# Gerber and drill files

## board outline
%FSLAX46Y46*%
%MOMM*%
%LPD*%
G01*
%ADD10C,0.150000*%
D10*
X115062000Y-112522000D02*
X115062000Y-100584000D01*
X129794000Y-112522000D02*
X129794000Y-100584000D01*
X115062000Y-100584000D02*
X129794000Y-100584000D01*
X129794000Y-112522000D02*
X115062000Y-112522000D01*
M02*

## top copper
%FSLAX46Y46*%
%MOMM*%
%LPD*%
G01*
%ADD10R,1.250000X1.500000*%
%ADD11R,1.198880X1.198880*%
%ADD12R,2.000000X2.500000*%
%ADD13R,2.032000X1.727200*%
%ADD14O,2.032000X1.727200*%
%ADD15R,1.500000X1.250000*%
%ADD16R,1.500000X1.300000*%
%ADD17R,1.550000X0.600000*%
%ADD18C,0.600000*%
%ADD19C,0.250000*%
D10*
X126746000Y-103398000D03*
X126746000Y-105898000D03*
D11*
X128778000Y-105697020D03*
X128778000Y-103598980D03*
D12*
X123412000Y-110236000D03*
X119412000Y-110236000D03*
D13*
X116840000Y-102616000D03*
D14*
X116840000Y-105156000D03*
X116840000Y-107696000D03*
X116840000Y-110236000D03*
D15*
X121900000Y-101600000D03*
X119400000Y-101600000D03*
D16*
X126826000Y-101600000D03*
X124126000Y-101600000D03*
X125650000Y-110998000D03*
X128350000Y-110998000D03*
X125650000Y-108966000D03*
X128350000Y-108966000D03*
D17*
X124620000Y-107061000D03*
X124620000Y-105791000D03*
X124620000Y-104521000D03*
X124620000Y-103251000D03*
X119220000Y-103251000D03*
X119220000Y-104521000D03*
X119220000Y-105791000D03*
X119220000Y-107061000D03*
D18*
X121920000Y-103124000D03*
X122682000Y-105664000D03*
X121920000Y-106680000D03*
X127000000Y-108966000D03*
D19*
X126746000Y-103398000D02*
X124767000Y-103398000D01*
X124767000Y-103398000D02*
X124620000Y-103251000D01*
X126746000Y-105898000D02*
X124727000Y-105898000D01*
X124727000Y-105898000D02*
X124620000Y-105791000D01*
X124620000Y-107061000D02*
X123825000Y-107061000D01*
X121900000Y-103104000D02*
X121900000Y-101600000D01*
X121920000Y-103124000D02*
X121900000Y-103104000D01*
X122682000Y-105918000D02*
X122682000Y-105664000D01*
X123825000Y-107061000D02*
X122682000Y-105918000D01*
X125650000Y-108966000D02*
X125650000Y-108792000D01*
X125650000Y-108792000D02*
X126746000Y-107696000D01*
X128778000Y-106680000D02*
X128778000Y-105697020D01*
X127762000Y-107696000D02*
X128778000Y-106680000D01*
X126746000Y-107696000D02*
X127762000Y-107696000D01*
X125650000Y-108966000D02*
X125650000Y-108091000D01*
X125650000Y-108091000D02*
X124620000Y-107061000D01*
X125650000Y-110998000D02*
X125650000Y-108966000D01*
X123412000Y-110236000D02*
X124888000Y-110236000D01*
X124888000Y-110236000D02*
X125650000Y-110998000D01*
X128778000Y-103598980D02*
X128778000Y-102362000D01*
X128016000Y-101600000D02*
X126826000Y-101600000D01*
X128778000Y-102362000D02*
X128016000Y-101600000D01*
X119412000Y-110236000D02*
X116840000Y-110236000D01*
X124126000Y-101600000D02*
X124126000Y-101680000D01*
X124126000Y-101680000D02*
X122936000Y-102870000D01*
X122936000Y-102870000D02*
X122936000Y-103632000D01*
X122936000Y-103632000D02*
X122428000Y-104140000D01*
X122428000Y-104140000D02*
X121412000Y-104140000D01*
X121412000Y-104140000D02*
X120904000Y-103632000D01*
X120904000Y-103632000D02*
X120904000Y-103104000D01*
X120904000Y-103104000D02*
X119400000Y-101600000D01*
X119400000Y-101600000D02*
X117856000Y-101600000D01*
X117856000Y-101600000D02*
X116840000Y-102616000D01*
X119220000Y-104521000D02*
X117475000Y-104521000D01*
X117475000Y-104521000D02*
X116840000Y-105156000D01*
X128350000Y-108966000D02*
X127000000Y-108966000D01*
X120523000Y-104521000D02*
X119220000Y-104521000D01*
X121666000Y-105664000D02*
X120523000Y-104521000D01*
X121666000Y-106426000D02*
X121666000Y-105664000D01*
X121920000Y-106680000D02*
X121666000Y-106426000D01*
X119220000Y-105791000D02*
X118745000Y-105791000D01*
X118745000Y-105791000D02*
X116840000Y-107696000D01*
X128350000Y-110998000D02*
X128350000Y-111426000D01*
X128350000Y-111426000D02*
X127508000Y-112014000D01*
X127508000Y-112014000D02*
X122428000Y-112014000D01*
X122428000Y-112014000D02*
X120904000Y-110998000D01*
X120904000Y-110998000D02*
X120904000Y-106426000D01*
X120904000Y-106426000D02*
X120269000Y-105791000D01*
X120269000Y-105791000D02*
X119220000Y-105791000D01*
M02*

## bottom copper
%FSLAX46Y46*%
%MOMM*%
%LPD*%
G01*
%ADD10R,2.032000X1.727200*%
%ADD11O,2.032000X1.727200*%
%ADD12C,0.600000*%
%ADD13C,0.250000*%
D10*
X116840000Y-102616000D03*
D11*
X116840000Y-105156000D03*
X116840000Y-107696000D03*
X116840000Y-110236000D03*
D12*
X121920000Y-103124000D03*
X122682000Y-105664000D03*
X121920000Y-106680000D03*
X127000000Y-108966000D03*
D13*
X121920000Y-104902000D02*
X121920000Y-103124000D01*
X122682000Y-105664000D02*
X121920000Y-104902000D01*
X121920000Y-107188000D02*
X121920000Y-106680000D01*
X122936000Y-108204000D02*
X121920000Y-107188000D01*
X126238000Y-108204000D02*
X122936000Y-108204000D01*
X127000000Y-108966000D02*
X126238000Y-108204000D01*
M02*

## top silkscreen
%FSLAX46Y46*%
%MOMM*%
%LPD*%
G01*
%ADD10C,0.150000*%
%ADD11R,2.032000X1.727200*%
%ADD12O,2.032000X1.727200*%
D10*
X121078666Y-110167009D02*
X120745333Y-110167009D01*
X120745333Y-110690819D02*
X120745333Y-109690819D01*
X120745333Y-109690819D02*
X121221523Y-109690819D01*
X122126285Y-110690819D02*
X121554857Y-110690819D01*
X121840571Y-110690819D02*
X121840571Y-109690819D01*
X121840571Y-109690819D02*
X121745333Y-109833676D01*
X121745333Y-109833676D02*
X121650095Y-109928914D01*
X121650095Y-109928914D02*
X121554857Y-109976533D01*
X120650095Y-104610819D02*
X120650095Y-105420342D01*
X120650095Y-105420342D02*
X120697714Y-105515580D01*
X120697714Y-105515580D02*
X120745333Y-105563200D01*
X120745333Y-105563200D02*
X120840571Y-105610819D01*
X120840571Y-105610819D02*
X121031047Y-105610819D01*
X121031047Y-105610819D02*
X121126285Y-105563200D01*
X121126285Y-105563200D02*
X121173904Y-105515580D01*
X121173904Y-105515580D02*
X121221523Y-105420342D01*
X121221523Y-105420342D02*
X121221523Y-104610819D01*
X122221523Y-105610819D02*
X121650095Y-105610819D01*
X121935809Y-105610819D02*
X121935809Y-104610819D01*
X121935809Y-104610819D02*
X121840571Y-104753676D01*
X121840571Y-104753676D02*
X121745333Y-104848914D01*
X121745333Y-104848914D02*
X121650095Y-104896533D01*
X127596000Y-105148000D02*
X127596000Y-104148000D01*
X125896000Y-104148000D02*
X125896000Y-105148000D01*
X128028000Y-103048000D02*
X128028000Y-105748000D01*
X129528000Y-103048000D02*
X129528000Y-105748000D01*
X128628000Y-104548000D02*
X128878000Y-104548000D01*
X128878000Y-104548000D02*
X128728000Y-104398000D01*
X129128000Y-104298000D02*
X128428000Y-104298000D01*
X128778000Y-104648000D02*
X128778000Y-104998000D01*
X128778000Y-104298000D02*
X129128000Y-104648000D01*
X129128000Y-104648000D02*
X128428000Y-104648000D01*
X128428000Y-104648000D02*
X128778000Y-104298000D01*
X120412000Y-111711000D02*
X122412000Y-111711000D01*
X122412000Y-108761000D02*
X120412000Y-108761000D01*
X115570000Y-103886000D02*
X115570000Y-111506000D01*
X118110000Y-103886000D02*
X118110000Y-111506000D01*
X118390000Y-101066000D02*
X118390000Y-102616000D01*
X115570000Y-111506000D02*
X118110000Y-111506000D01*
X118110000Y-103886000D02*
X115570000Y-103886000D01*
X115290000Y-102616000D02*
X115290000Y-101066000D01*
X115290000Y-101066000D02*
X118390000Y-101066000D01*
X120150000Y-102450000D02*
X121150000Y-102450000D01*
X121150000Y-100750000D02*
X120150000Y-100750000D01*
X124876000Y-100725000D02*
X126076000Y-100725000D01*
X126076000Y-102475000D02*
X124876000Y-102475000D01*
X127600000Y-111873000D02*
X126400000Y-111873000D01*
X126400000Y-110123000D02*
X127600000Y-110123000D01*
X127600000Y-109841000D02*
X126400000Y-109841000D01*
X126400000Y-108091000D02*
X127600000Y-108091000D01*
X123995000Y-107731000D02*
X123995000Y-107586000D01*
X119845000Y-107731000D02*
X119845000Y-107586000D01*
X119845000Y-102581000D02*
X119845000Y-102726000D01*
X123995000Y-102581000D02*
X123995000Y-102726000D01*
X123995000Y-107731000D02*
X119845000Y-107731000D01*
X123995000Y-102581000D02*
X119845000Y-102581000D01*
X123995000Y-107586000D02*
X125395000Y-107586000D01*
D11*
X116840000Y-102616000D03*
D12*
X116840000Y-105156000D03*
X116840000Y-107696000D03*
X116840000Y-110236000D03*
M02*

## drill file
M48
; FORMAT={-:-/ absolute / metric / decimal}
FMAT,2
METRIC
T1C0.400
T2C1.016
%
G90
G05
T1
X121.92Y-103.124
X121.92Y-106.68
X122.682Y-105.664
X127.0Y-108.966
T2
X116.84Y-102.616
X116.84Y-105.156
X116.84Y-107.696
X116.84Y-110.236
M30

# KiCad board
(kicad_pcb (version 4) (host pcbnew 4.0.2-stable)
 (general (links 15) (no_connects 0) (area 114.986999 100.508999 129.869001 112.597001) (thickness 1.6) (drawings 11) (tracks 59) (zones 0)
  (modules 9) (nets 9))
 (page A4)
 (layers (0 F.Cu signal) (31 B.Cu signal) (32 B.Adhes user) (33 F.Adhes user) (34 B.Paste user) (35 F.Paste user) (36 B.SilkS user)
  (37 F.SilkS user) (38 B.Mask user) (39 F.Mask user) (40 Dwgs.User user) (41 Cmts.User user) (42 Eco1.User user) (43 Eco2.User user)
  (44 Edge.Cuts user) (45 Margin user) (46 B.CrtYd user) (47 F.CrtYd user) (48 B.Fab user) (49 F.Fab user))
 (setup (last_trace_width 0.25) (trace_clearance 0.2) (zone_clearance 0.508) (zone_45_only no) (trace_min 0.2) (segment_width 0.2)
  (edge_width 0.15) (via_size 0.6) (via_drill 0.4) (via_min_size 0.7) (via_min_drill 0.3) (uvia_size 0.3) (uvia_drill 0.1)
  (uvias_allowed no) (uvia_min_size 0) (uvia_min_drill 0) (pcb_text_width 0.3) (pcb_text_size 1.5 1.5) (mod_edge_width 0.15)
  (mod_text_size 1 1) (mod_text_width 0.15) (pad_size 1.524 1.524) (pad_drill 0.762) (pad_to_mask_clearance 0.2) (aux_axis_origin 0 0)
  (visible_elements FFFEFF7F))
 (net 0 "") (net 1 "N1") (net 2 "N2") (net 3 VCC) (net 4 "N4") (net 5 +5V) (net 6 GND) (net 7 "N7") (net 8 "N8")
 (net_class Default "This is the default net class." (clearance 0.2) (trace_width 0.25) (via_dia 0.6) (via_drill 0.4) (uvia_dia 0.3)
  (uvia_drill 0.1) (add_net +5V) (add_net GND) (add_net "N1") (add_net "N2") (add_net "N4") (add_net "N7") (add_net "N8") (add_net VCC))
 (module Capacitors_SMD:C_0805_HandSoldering (layer F.Cu) (at 126.746 104.648 270)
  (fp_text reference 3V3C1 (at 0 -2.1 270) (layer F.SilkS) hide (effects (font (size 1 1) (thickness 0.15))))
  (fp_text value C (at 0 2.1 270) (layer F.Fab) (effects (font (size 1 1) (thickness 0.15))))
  (fp_line (start 0.5 -0.85) (end -0.5 -0.85) (layer F.SilkS) (width 0.15))
  (fp_line (start -0.5 0.85) (end 0.5 0.85) (layer F.SilkS) (width 0.15))
  (pad 1 smd rect (at -1.25 0 270) (size 1.5 1.25) (layers F.Cu F.Paste F.Mask) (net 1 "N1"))
  (pad 2 smd rect (at 1.25 0 270) (size 1.5 1.25) (layers F.Cu F.Paste F.Mask) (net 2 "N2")))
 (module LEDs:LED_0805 (layer F.Cu) (at 128.778 104.648 270)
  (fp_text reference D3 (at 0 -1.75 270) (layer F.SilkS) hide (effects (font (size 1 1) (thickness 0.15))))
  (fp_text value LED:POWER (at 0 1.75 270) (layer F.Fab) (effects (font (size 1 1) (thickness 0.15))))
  (fp_line (start -1.6 0.75) (end 1.1 0.75) (layer F.SilkS) (width 0.15))
  (fp_line (start -1.6 -0.75) (end 1.1 -0.75) (layer F.SilkS) (width 0.15))
  (fp_line (start -0.1 0.15) (end -0.1 -0.1) (layer F.SilkS) (width 0.15))
  (fp_line (start -0.1 -0.1) (end -0.25 0.05) (layer F.SilkS) (width 0.15))
  (fp_line (start -0.35 -0.35) (end -0.35 0.35) (layer F.SilkS) (width 0.15))
  (fp_line (start 0 0) (end 0.35 0) (layer F.SilkS) (width 0.15))
  (fp_line (start -0.35 0) (end 0 -0.35) (layer F.SilkS) (width 0.15))
  (fp_line (start 0 -0.35) (end 0 0.35) (layer F.SilkS) (width 0.15))
  (fp_line (start 0 0.35) (end -0.35 0) (layer F.SilkS) (width 0.15))
  (pad 2 smd rect (at 1.04902 0 90) (size 1.19888 1.19888) (layers F.Cu F.Paste F.Mask) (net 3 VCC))
  (pad 1 smd rect (at -1.04902 0 90) (size 1.19888 1.19888) (layers F.Cu F.Paste F.Mask) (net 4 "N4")))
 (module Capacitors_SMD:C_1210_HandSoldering (layer F.Cu) (at 121.412 110.236 180)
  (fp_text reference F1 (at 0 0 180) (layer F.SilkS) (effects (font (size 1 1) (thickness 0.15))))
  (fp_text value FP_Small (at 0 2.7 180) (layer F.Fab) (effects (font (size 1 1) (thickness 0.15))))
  (fp_line (start 1 -1.475) (end -1 -1.475) (layer F.SilkS) (width 0.15))
  (fp_line (start -1 1.475) (end 1 1.475) (layer F.SilkS) (width 0.15))
  (pad 1 smd rect (at -2 0 180) (size 2 2.5) (layers F.Cu F.Paste F.Mask) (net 3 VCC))
  (pad 2 smd rect (at 2 0 180) (size 2 2.5) (layers F.Cu F.Paste F.Mask) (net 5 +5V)))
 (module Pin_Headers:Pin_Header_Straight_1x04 (layer F.Cu) (at 116.84 102.616)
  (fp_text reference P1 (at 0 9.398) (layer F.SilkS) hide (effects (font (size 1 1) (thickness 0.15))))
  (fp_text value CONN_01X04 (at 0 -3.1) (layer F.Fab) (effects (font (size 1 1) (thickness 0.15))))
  (fp_line (start -1.27 1.27) (end -1.27 8.89) (layer F.SilkS) (width 0.15))
  (fp_line (start 1.27 1.27) (end 1.27 8.89) (layer F.SilkS) (width 0.15))
  (fp_line (start 1.55 -1.55) (end 1.55 0) (layer F.SilkS) (width 0.15))
  (fp_line (start -1.27 8.89) (end 1.27 8.89) (layer F.SilkS) (width 0.15))
  (fp_line (start 1.27 1.27) (end -1.27 1.27) (layer F.SilkS) (width 0.15))
  (fp_line (start -1.55 0) (end -1.55 -1.55) (layer F.SilkS) (width 0.15))
  (fp_line (start -1.55 -1.55) (end 1.55 -1.55) (layer F.SilkS) (width 0.15))
  (pad 1 thru_hole rect (at 0 0) (size 2.032 1.7272) (drill 1.016) (layers *.Cu *.Mask F.SilkS) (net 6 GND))
  (pad 2 thru_hole oval (at 0 2.54) (size 2.032 1.7272) (drill 1.016) (layers *.Cu *.Mask F.SilkS) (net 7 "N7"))
  (pad 3 thru_hole oval (at 0 5.08) (size 2.032 1.7272) (drill 1.016) (layers *.Cu *.Mask F.SilkS) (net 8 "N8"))
  (pad 4 thru_hole oval (at 0 7.62) (size 2.032 1.7272) (drill 1.016) (layers *.Cu *.Mask F.SilkS) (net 5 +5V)))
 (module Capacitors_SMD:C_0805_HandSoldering (layer F.Cu) (at 120.65 101.6 180)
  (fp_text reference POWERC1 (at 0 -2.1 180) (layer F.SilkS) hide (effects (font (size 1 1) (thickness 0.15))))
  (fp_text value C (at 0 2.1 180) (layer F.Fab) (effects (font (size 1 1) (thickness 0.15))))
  (fp_line (start 0.5 -0.85) (end -0.5 -0.85) (layer F.SilkS) (width 0.15))
  (fp_line (start -0.5 0.85) (end 0.5 0.85) (layer F.SilkS) (width 0.15))
  (pad 1 smd rect (at -1.25 0 180) (size 1.5 1.25) (layers F.Cu F.Paste F.Mask) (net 3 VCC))
  (pad 2 smd rect (at 1.25 0 180) (size 1.5 1.25) (layers F.Cu F.Paste F.Mask) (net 6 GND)))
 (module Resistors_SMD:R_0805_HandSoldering (layer F.Cu) (at 125.476 101.6 180)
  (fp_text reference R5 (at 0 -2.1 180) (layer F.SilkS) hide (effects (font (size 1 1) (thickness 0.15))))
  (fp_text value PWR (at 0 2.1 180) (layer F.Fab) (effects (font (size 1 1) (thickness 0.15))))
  (fp_line (start 0.6 0.875) (end -0.6 0.875) (layer F.SilkS) (width 0.15))
  (fp_line (start -0.6 -0.875) (end 0.6 -0.875) (layer F.SilkS) (width 0.15))
  (pad 1 smd rect (at -1.35 0 180) (size 1.5 1.3) (layers F.Cu F.Paste F.Mask) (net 4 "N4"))
  (pad 2 smd rect (at 1.35 0 180) (size 1.5 1.3) (layers F.Cu F.Paste F.Mask) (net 6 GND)))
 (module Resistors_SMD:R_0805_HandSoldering (layer F.Cu) (at 127 110.998)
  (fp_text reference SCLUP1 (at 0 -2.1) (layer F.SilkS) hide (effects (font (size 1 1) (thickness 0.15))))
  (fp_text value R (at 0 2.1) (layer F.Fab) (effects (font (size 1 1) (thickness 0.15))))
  (fp_line (start 0.6 0.875) (end -0.6 0.875) (layer F.SilkS) (width 0.15))
  (fp_line (start -0.6 -0.875) (end 0.6 -0.875) (layer F.SilkS) (width 0.15))
  (pad 1 smd rect (at -1.35 0) (size 1.5 1.3) (layers F.Cu F.Paste F.Mask) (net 3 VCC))
  (pad 2 smd rect (at 1.35 0) (size 1.5 1.3) (layers F.Cu F.Paste F.Mask) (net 8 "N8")))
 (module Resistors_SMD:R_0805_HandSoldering (layer F.Cu) (at 127 108.966)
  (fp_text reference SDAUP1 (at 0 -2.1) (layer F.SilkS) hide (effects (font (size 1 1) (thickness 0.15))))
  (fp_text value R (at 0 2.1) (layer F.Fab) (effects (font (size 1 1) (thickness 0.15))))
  (fp_line (start 0.6 0.875) (end -0.6 0.875) (layer F.SilkS) (width 0.15))
  (fp_line (start -0.6 -0.875) (end 0.6 -0.875) (layer F.SilkS) (width 0.15))
  (pad 1 smd rect (at -1.35 0) (size 1.5 1.3) (layers F.Cu F.Paste F.Mask) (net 3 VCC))
  (pad 2 smd rect (at 1.35 0) (size 1.5 1.3) (layers F.Cu F.Paste F.Mask) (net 7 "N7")))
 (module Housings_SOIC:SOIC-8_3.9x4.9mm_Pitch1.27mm (layer F.Cu) (at 121.92 105.156 180)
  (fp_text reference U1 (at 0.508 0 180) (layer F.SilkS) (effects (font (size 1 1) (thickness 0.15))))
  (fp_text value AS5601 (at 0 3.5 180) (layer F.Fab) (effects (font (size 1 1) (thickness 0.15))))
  (fp_line (start -2.075 -2.575) (end -2.075 -2.43) (layer F.SilkS) (width 0.15))
  (fp_line (start 2.075 -2.575) (end 2.075 -2.43) (layer F.SilkS) (width 0.15))
  (fp_line (start 2.075 2.575) (end 2.075 2.43) (layer F.SilkS) (width 0.15))
  (fp_line (start -2.075 2.575) (end -2.075 2.43) (layer F.SilkS) (width 0.15))
  (fp_line (start -2.075 -2.575) (end 2.075 -2.575) (layer F.SilkS) (width 0.15))
  (fp_line (start -2.075 2.575) (end 2.075 2.575) (layer F.SilkS) (width 0.15))
  (fp_line (start -2.075 -2.43) (end -3.475 -2.43) (layer F.SilkS) (width 0.15))
  (pad 1 smd rect (at -2.7 -1.905 180) (size 1.55 0.6) (layers F.Cu F.Paste F.Mask) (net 3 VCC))
  (pad 2 smd rect (at -2.7 -0.635 180) (size 1.55 0.6) (layers F.Cu F.Paste F.Mask) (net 2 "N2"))
  (pad 3 smd rect (at -2.7 0.635 180) (size 1.55 0.6) (layers F.Cu F.Paste F.Mask))
  (pad 4 smd rect (at -2.7 1.905 180) (size 1.55 0.6) (layers F.Cu F.Paste F.Mask) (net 1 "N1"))
  (pad 5 smd rect (at 2.7 1.905 180) (size 1.55 0.6) (layers F.Cu F.Paste F.Mask))
  (pad 6 smd rect (at 2.7 0.635 180) (size 1.55 0.6) (layers F.Cu F.Paste F.Mask) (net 7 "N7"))
  (pad 7 smd rect (at 2.7 -0.635 180) (size 1.55 0.6) (layers F.Cu F.Paste F.Mask) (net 8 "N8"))
  (pad 8 smd rect (at 2.7 -1.905 180) (size 1.55 0.6) (layers F.Cu F.Paste F.Mask)))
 (gr_line (start 115.062 112.522) (end 115.062 100.584) (angle 90) (layer Edge.Cuts) (width 0.15))
 (gr_line (start 129.794 112.522) (end 129.794 100.584) (angle 90) (layer Edge.Cuts) (width 0.15))
 (gr_line (start 115.062 100.584) (end 129.794 100.584) (angle 90) (layer Edge.Cuts) (width 0.15))
 (gr_line (start 129.794 112.522) (end 115.062 112.522) (angle 90) (layer Edge.Cuts) (width 0.15))
 (segment (start 126.746 103.398) (end 124.767 103.398) (width 0.25) (layer F.Cu) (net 1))
 (segment (start 124.767 103.398) (end 124.62 103.251) (width 0.25) (layer F.Cu) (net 1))
 (segment (start 126.746 105.898) (end 124.727 105.898) (width 0.25) (layer F.Cu) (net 2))
 (segment (start 124.727 105.898) (end 124.62 105.791) (width 0.25) (layer F.Cu) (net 2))
 (segment (start 124.62 107.061) (end 123.825 107.061) (width 0.25) (layer F.Cu) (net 3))
 (segment (start 121.9 103.104) (end 121.9 101.6) (width 0.25) (layer F.Cu) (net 3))
 (segment (start 121.92 103.124) (end 121.9 103.104) (width 0.25) (layer F.Cu) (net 3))
 (segment (start 121.92 104.902) (end 121.92 103.124) (width 0.25) (layer B.Cu) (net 3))
 (segment (start 122.682 105.664) (end 121.92 104.902) (width 0.25) (layer B.Cu) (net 3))
 (segment (start 122.682 105.918) (end 122.682 105.664) (width 0.25) (layer F.Cu) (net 3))
 (segment (start 123.825 107.061) (end 122.682 105.918) (width 0.25) (layer F.Cu) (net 3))
 (segment (start 125.65 108.966) (end 125.65 108.792) (width 0.25) (layer F.Cu) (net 3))
 (segment (start 125.65 108.792) (end 126.746 107.696) (width 0.25) (layer F.Cu) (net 3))
 (segment (start 128.778 106.68) (end 128.778 105.69702) (width 0.25) (layer F.Cu) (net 3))
 (segment (start 127.762 107.696) (end 128.778 106.68) (width 0.25) (layer F.Cu) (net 3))
 (segment (start 126.746 107.696) (end 127.762 107.696) (width 0.25) (layer F.Cu) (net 3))
 (segment (start 125.65 108.966) (end 125.65 108.091) (width 0.25) (layer F.Cu) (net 3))
 (segment (start 125.65 108.091) (end 124.62 107.061) (width 0.25) (layer F.Cu) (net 3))
 (segment (start 125.65 110.998) (end 125.65 108.966) (width 0.25) (layer F.Cu) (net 3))
 (segment (start 123.412 110.236) (end 124.888 110.236) (width 0.25) (layer F.Cu) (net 3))
 (segment (start 124.888 110.236) (end 125.65 110.998) (width 0.25) (layer F.Cu) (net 3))
 (segment (start 128.778 103.59898) (end 128.778 102.362) (width 0.25) (layer F.Cu) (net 4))
 (segment (start 128.016 101.6) (end 126.826 101.6) (width 0.25) (layer F.Cu) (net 4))
 (segment (start 128.778 102.362) (end 128.016 101.6) (width 0.25) (layer F.Cu) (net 4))
 (segment (start 119.412 110.236) (end 116.84 110.236) (width 0.25) (layer F.Cu) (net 5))
 (segment (start 124.126 101.6) (end 124.126 101.68) (width 0.25) (layer F.Cu) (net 6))
 (segment (start 124.126 101.68) (end 122.936 102.87) (width 0.25) (layer F.Cu) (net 6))
 (segment (start 122.936 102.87) (end 122.936 103.632) (width 0.25) (layer F.Cu) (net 6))
 (segment (start 122.936 103.632) (end 122.428 104.14) (width 0.25) (layer F.Cu) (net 6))
 (segment (start 122.428 104.14) (end 121.412 104.14) (width 0.25) (layer F.Cu) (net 6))
 (segment (start 121.412 104.14) (end 120.904 103.632) (width 0.25) (layer F.Cu) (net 6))
 (segment (start 120.904 103.632) (end 120.904 103.104) (width 0.25) (layer F.Cu) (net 6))
 (segment (start 120.904 103.104) (end 119.4 101.6) (width 0.25) (layer F.Cu) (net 6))
 (segment (start 119.4 101.6) (end 117.856 101.6) (width 0.25) (layer F.Cu) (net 6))
 (segment (start 117.856 101.6) (end 116.84 102.616) (width 0.25) (layer F.Cu) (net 6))
 (segment (start 119.22 104.521) (end 117.475 104.521) (width 0.25) (layer F.Cu) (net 7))
 (segment (start 117.475 104.521) (end 116.84 105.156) (width 0.25) (layer F.Cu) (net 7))
 (segment (start 128.35 108.966) (end 127 108.966) (width 0.25) (layer F.Cu) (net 7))
 (segment (start 120.523 104.521) (end 119.22 104.521) (width 0.25) (layer F.Cu) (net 7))
 (segment (start 121.666 105.664) (end 120.523 104.521) (width 0.25) (layer F.Cu) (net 7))
 (segment (start 121.666 106.426) (end 121.666 105.664) (width 0.25) (layer F.Cu) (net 7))
 (segment (start 121.92 106.68) (end 121.666 106.426) (width 0.25) (layer F.Cu) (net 7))
 (segment (start 121.92 107.188) (end 121.92 106.68) (width 0.25) (layer B.Cu) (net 7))
 (segment (start 122.936 108.204) (end 121.92 107.188) (width 0.25) (layer B.Cu) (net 7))
 (segment (start 126.238 108.204) (end 122.936 108.204) (width 0.25) (layer B.Cu) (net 7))
 (segment (start 127 108.966) (end 126.238 108.204) (width 0.25) (layer B.Cu) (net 7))
 (segment (start 119.22 105.791) (end 118.745 105.791) (width 0.25) (layer F.Cu) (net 8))
 (segment (start 118.745 105.791) (end 116.84 107.696) (width 0.25) (layer F.Cu) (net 8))
 (segment (start 128.35 110.998) (end 128.35 111.426) (width 0.25) (layer F.Cu) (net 8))
 (segment (start 128.35 111.426) (end 127.508 112.014) (width 0.25) (layer F.Cu) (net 8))
 (segment (start 127.508 112.014) (end 122.428 112.014) (width 0.25) (layer F.Cu) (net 8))
 (segment (start 122.428 112.014) (end 120.904 110.998) (width 0.25) (layer F.Cu) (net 8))
 (segment (start 120.904 110.998) (end 120.904 106.426) (width 0.25) (layer F.Cu) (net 8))
 (segment (start 120.904 106.426) (end 120.269 105.791) (width 0.25) (layer F.Cu) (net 8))
 (segment (start 120.269 105.791) (end 119.22 105.791) (width 0.25) (layer F.Cu) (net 8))
 (via (at 121.92 103.124) (size 0.6) (drill 0.4) (layers F.Cu B.Cu) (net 3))
 (via (at 122.682 105.664) (size 0.6) (drill 0.4) (layers F.Cu B.Cu) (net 3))
 (via (at 121.92 106.68) (size 0.6) (drill 0.4) (layers F.Cu B.Cu) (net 7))
 (via (at 127 108.966) (size 0.6) (drill 0.4) (layers F.Cu B.Cu) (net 7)))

